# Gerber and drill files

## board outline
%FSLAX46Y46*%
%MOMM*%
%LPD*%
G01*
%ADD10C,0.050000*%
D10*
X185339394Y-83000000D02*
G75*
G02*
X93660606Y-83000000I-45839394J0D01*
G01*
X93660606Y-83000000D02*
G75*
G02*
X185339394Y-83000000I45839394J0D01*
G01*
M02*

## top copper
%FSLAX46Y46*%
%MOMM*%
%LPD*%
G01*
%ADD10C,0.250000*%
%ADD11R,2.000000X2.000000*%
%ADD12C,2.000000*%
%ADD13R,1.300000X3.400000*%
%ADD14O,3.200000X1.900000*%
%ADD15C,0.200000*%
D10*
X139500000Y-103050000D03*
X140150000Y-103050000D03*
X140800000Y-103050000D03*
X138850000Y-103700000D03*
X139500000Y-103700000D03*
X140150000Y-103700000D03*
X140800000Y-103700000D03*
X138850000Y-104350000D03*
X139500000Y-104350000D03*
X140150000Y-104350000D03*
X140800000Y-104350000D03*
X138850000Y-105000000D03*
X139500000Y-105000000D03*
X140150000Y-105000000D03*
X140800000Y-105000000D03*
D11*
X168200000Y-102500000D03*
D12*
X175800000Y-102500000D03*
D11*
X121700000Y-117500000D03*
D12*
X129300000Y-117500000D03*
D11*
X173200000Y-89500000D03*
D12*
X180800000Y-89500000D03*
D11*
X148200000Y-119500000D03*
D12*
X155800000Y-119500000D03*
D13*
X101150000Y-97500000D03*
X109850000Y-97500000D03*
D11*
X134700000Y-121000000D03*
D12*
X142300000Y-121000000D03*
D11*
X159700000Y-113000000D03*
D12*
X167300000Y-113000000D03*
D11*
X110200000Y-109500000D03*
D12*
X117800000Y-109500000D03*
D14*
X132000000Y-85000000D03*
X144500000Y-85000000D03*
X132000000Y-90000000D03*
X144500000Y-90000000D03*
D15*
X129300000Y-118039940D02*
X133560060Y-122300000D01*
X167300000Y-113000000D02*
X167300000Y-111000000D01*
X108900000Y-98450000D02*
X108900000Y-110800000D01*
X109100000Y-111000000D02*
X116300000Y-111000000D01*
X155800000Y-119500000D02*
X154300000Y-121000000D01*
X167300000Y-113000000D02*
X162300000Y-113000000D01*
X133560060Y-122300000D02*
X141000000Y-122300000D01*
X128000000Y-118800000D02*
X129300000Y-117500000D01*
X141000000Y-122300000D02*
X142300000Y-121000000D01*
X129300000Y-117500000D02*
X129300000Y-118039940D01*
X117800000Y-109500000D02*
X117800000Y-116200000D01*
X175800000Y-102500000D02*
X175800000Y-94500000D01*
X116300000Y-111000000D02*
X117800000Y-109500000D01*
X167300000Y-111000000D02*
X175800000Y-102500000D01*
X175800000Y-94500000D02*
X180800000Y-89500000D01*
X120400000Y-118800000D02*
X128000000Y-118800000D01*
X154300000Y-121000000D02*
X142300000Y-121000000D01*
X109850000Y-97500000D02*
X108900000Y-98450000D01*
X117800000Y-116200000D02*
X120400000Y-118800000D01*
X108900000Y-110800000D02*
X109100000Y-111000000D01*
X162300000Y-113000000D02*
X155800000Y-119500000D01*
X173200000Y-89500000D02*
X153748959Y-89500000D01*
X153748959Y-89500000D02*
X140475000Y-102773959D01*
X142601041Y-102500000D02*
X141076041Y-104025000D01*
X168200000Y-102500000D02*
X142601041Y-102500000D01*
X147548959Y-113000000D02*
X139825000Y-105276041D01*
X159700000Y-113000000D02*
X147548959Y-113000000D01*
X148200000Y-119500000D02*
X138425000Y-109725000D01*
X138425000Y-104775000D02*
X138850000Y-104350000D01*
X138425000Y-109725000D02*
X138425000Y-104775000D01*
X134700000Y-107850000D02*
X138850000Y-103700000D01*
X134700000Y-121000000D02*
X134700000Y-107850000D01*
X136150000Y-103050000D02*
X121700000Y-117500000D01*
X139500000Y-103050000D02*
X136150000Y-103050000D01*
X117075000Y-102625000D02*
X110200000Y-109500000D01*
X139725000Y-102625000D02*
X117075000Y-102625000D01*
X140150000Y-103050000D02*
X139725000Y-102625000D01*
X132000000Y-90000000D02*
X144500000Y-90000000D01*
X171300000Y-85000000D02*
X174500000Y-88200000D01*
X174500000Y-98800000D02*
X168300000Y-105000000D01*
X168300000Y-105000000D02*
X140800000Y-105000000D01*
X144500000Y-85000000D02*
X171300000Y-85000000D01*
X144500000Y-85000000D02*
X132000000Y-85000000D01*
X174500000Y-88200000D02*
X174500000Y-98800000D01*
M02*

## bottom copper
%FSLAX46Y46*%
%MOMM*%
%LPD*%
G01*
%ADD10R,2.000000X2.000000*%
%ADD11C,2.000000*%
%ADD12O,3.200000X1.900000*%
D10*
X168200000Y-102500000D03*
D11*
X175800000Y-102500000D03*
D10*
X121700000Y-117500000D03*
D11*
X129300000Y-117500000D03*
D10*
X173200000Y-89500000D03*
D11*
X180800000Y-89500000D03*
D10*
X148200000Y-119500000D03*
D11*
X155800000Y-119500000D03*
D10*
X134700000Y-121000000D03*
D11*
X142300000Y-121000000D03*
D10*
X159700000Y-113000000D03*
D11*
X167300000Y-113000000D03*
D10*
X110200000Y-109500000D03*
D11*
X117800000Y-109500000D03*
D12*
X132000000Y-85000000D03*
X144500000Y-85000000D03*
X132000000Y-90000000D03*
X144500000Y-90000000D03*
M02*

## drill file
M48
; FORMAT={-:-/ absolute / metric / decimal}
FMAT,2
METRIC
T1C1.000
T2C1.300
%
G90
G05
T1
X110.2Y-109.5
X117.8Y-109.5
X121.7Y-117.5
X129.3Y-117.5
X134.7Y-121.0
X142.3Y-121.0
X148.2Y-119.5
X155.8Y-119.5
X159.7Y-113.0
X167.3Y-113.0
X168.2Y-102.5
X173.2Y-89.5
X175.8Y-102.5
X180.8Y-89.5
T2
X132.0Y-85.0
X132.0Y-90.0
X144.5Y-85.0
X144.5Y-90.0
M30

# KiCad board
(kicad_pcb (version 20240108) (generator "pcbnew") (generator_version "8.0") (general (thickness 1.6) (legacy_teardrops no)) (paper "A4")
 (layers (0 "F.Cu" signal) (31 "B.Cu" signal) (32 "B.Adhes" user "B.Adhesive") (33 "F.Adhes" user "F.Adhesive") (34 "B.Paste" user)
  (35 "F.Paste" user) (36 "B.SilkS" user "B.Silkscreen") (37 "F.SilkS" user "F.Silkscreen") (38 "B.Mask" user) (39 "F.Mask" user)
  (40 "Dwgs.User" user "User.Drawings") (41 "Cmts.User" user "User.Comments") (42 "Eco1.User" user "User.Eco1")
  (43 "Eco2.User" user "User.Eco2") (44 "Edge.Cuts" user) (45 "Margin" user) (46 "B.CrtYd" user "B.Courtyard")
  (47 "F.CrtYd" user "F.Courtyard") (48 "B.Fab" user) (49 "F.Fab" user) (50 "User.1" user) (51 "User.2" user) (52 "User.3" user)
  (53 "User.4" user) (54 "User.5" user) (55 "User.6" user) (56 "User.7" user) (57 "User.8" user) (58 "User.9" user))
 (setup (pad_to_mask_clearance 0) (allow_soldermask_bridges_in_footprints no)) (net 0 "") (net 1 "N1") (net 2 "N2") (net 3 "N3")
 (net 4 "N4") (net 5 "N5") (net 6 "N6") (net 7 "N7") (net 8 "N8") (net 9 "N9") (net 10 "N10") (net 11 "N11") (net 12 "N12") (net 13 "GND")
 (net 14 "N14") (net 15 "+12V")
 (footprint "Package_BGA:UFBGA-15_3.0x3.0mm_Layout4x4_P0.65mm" (layer "F.Cu") (at 139.825 104.025)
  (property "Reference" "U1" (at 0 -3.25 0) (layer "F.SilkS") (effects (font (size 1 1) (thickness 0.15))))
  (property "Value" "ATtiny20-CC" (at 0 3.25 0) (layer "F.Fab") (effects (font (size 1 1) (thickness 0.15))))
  (pad "A2" smd circle (at -0.325 -0.975) (size 0.25 0.25) (layers "F.Cu" "F.Paste" "F.Mask") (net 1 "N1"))
  (pad "A3" smd circle (at 0.325 -0.975) (size 0.25 0.25) (layers "F.Cu" "F.Paste" "F.Mask") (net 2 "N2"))
  (pad "A4" smd circle (at 0.975 -0.975) (size 0.25 0.25) (layers "F.Cu" "F.Paste" "F.Mask") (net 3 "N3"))
  (pad "B1" smd circle (at -0.975 -0.325) (size 0.25 0.25) (layers "F.Cu" "F.Paste" "F.Mask") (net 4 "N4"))
  (pad "B2" smd circle (at -0.325 -0.325) (size 0.25 0.25) (layers "F.Cu" "F.Paste" "F.Mask") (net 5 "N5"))
  (pad "B3" smd circle (at 0.325 -0.325) (size 0.25 0.25) (layers "F.Cu" "F.Paste" "F.Mask") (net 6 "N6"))
  (pad "B4" smd circle (at 0.975 -0.325) (size 0.25 0.25) (layers "F.Cu" "F.Paste" "F.Mask") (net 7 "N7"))
  (pad "C1" smd circle (at -0.975 0.325) (size 0.25 0.25) (layers "F.Cu" "F.Paste" "F.Mask") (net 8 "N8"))
  (pad "C2" smd circle (at -0.325 0.325) (size 0.25 0.25) (layers "F.Cu" "F.Paste" "F.Mask") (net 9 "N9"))
  (pad "C3" smd circle (at 0.325 0.325) (size 0.25 0.25) (layers "F.Cu" "F.Paste" "F.Mask") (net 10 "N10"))
  (pad "C4" smd circle (at 0.975 0.325) (size 0.25 0.25) (layers "F.Cu" "F.Paste" "F.Mask") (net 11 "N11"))
  (pad "D1" smd circle (at -0.975 0.975) (size 0.25 0.25) (layers "F.Cu" "F.Paste" "F.Mask") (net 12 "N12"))
  (pad "D2" smd circle (at -0.325 0.975) (size 0.25 0.25) (layers "F.Cu" "F.Paste" "F.Mask") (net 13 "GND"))
  (pad "D3" smd circle (at 0.325 0.975) (size 0.25 0.25) (layers "F.Cu" "F.Paste" "F.Mask") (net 13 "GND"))
  (pad "D4" smd circle (at 0.975 0.975) (size 0.25 0.25) (layers "F.Cu" "F.Paste" "F.Mask") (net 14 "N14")))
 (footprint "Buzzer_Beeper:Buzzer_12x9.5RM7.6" (layer "F.Cu") (at 168.2 102.5)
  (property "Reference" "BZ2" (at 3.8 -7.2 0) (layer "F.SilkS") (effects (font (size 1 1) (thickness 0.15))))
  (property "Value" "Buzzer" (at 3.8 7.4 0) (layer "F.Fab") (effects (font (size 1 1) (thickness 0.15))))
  (pad "1" thru_hole rect (at 0 0) (size 2 2) (drill 1) (layers "*.Cu" "*.Mask") (remove_unused_layers no) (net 10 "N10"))
  (pad "2" thru_hole circle (at 7.6 0) (size 2 2) (drill 1) (layers "*.Cu" "*.Mask") (remove_unused_layers no) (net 13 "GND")))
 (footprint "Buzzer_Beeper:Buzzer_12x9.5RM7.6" (layer "F.Cu") (at 121.7 117.5)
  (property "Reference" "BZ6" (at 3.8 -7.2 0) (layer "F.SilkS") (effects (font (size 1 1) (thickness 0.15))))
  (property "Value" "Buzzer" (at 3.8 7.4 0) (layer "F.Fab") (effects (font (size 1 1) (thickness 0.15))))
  (pad "1" thru_hole rect (at 0 0) (size 2 2) (drill 1) (layers "*.Cu" "*.Mask") (remove_unused_layers no) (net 1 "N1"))
  (pad "2" thru_hole circle (at 7.6 0) (size 2 2) (drill 1) (layers "*.Cu" "*.Mask") (remove_unused_layers no) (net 13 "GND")))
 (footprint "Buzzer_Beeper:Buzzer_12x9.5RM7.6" (layer "F.Cu") (at 173.2 89.5)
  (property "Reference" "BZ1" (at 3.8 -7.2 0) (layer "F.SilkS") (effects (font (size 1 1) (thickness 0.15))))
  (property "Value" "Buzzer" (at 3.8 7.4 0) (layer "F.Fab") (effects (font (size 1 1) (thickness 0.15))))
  (pad "1" thru_hole rect (at 0 0) (size 2 2) (drill 1) (layers "*.Cu" "*.Mask") (remove_unused_layers no) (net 12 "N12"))
  (pad "2" thru_hole circle (at 7.6 0) (size 2 2) (drill 1) (layers "*.Cu" "*.Mask") (remove_unused_layers no) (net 13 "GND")))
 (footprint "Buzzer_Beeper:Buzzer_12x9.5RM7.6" (layer "F.Cu") (at 148.2 119.5)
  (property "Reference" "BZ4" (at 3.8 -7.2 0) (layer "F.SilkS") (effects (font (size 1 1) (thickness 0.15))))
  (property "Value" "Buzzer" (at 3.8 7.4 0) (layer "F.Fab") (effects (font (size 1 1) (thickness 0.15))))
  (pad "1" thru_hole rect (at 0 0) (size 2 2) (drill 1) (layers "*.Cu" "*.Mask") (remove_unused_layers no) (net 8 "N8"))
  (pad "2" thru_hole circle (at 7.6 0) (size 2 2) (drill 1) (layers "*.Cu" "*.Mask") (remove_unused_layers no) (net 13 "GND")))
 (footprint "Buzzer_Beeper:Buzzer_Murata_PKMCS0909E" (layer "F.Cu") (at 105.5 97.5)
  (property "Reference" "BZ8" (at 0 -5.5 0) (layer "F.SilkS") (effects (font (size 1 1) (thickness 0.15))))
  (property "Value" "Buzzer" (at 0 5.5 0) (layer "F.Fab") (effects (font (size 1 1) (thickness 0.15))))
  (pad "1" smd rect (at -4.35 0) (size 1.3 3.4) (layers "F.Cu" "F.Paste" "F.Mask") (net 5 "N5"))
  (pad "2" smd rect (at 4.35 0) (size 1.3 3.4) (layers "F.Cu" "F.Paste" "F.Mask") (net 13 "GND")))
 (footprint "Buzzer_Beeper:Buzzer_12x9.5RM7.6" (layer "F.Cu") (at 134.7 121)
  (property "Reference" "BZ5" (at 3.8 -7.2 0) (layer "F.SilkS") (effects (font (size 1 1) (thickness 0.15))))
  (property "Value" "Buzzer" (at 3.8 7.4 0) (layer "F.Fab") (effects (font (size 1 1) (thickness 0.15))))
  (pad "1" thru_hole rect (at 0 0) (size 2 2) (drill 1) (layers "*.Cu" "*.Mask") (remove_unused_layers no) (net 4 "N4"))
  (pad "2" thru_hole circle (at 7.6 0) (size 2 2) (drill 1) (layers "*.Cu" "*.Mask") (remove_unused_layers no) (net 13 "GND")))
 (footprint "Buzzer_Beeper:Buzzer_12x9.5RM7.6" (layer "F.Cu") (at 159.7 113)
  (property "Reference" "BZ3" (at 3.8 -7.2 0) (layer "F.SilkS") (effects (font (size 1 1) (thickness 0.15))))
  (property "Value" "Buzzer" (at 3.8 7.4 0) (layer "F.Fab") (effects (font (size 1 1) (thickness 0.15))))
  (pad "1" thru_hole rect (at 0 0) (size 2 2) (drill 1) (layers "*.Cu" "*.Mask") (remove_unused_layers no) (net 9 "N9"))
  (pad "2" thru_hole circle (at 7.6 0) (size 2 2) (drill 1) (layers "*.Cu" "*.Mask") (remove_unused_layers no) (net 13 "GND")))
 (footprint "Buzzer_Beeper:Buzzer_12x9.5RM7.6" (layer "F.Cu") (at 110.2 109.5)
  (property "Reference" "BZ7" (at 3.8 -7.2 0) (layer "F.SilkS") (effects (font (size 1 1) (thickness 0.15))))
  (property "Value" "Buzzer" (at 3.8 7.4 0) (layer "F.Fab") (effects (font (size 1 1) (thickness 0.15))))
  (pad "1" thru_hole rect (at 0 0) (size 2 2) (drill 1) (layers "*.Cu" "*.Mask") (remove_unused_layers no) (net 2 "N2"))
  (pad "2" thru_hole circle (at 7.6 0) (size 2 2) (drill 1) (layers "*.Cu" "*.Mask") (remove_unused_layers no) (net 13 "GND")))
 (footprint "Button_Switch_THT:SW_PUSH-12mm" (layer "F.Cu") (at 132 85)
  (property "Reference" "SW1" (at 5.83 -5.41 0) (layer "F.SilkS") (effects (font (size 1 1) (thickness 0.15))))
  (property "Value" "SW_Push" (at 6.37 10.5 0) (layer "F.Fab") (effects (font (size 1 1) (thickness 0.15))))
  (pad "1" thru_hole oval (at 0 0) (size 3.2 1.9) (drill 1.3) (layers "*.Cu" "*.Mask") (remove_unused_layers no) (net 14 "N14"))
  (pad "1" thru_hole oval (at 12.5 0) (size 3.2 1.9) (drill 1.3) (layers "*.Cu" "*.Mask") (remove_unused_layers no) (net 14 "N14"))
  (pad "2" thru_hole oval (at 0 5) (size 3.2 1.9) (drill 1.3) (layers "*.Cu" "*.Mask") (remove_unused_layers no) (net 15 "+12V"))
  (pad "2" thru_hole oval (at 12.5 5) (size 3.2 1.9) (drill 1.3) (layers "*.Cu" "*.Mask") (remove_unused_layers no) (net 15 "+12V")))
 (gr_circle (center 139.5 83) (end 175 54) (stroke (width 0.05) (type default)) (fill none) (layer "Edge.Cuts"))
 (segment (start 129.3 118.03994) (end 133.56006 122.3) (width 0.2) (layer "F.Cu") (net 13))
 (segment (start 167.3 113) (end 167.3 111) (width 0.2) (layer "F.Cu") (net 13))
 (segment (start 108.9 98.45) (end 108.9 110.8) (width 0.2) (layer "F.Cu") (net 13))
 (segment (start 109.1 111) (end 116.3 111) (width 0.2) (layer "F.Cu") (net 13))
 (segment (start 155.8 119.5) (end 154.3 121) (width 0.2) (layer "F.Cu") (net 13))
 (segment (start 167.3 113) (end 162.3 113) (width 0.2) (layer "F.Cu") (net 13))
 (segment (start 133.56006 122.3) (end 141 122.3) (width 0.2) (layer "F.Cu") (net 13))
 (segment (start 128 118.8) (end 129.3 117.5) (width 0.2) (layer "F.Cu") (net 13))
 (segment (start 141 122.3) (end 142.3 121) (width 0.2) (layer "F.Cu") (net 13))
 (segment (start 129.3 117.5) (end 129.3 118.03994) (width 0.2) (layer "F.Cu") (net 13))
 (segment (start 117.8 109.5) (end 117.8 116.2) (width 0.2) (layer "F.Cu") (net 13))
 (segment (start 175.8 102.5) (end 175.8 94.5) (width 0.2) (layer "F.Cu") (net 13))
 (segment (start 116.3 111) (end 117.8 109.5) (width 0.2) (layer "F.Cu") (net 13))
 (segment (start 167.3 111) (end 175.8 102.5) (width 0.2) (layer "F.Cu") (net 13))
 (segment (start 175.8 94.5) (end 180.8 89.5) (width 0.2) (layer "F.Cu") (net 13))
 (segment (start 120.4 118.8) (end 128 118.8) (width 0.2) (layer "F.Cu") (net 13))
 (segment (start 154.3 121) (end 142.3 121) (width 0.2) (layer "F.Cu") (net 13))
 (segment (start 109.85 97.5) (end 108.9 98.45) (width 0.2) (layer "F.Cu") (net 13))
 (segment (start 117.8 116.2) (end 120.4 118.8) (width 0.2) (layer "F.Cu") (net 13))
 (segment (start 108.9 110.8) (end 109.1 111) (width 0.2) (layer "F.Cu") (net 13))
 (segment (start 162.3 113) (end 155.8 119.5) (width 0.2) (layer "F.Cu") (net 13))
 (segment (start 173.2 89.5) (end 153.748959 89.5) (width 0.2) (layer "F.Cu") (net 12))
 (segment (start 153.748959 89.5) (end 140.475 102.773959) (width 0.2) (layer "F.Cu") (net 12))
 (segment (start 142.601041 102.5) (end 141.076041 104.025) (width 0.2) (layer "F.Cu") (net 10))
 (segment (start 168.2 102.5) (end 142.601041 102.5) (width 0.2) (layer "F.Cu") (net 10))
 (segment (start 147.548959 113) (end 139.825 105.276041) (width 0.2) (layer "F.Cu") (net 9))
 (segment (start 159.7 113) (end 147.548959 113) (width 0.2) (layer "F.Cu") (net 9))
 (segment (start 148.2 119.5) (end 138.425 109.725) (width 0.2) (layer "F.Cu") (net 8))
 (segment (start 138.425 104.775) (end 138.85 104.35) (width 0.2) (layer "F.Cu") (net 8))
 (segment (start 138.425 109.725) (end 138.425 104.775) (width 0.2) (layer "F.Cu") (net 8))
 (segment (start 134.7 107.85) (end 138.85 103.7) (width 0.2) (layer "F.Cu") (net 4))
 (segment (start 134.7 121) (end 134.7 107.85) (width 0.2) (layer "F.Cu") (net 4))
 (segment (start 136.15 103.05) (end 121.7 117.5) (width 0.2) (layer "F.Cu") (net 1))
 (segment (start 139.5 103.05) (end 136.15 103.05) (width 0.2) (layer "F.Cu") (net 1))
 (segment (start 117.075 102.625) (end 110.2 109.5) (width 0.2) (layer "F.Cu") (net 2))
 (segment (start 139.725 102.625) (end 117.075 102.625) (width 0.2) (layer "F.Cu") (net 2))
 (segment (start 140.15 103.05) (end 139.725 102.625) (width 0.2) (layer "F.Cu") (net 2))
 (segment (start 132 90) (end 144.5 90) (width 0.2) (layer "F.Cu") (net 15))
 (segment (start 171.3 85) (end 174.5 88.2) (width 0.2) (layer "F.Cu") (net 14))
 (segment (start 174.5 98.8) (end 168.3 105) (width 0.2) (layer "F.Cu") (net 14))
 (segment (start 168.3 105) (end 140.8 105) (width 0.2) (layer "F.Cu") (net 14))
 (segment (start 144.5 85) (end 171.3 85) (width 0.2) (layer "F.Cu") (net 14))
 (segment (start 144.5 85) (end 132 85) (width 0.2) (layer "F.Cu") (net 14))
 (segment (start 174.5 88.2) (end 174.5 98.8) (width 0.2) (layer "F.Cu") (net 14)))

